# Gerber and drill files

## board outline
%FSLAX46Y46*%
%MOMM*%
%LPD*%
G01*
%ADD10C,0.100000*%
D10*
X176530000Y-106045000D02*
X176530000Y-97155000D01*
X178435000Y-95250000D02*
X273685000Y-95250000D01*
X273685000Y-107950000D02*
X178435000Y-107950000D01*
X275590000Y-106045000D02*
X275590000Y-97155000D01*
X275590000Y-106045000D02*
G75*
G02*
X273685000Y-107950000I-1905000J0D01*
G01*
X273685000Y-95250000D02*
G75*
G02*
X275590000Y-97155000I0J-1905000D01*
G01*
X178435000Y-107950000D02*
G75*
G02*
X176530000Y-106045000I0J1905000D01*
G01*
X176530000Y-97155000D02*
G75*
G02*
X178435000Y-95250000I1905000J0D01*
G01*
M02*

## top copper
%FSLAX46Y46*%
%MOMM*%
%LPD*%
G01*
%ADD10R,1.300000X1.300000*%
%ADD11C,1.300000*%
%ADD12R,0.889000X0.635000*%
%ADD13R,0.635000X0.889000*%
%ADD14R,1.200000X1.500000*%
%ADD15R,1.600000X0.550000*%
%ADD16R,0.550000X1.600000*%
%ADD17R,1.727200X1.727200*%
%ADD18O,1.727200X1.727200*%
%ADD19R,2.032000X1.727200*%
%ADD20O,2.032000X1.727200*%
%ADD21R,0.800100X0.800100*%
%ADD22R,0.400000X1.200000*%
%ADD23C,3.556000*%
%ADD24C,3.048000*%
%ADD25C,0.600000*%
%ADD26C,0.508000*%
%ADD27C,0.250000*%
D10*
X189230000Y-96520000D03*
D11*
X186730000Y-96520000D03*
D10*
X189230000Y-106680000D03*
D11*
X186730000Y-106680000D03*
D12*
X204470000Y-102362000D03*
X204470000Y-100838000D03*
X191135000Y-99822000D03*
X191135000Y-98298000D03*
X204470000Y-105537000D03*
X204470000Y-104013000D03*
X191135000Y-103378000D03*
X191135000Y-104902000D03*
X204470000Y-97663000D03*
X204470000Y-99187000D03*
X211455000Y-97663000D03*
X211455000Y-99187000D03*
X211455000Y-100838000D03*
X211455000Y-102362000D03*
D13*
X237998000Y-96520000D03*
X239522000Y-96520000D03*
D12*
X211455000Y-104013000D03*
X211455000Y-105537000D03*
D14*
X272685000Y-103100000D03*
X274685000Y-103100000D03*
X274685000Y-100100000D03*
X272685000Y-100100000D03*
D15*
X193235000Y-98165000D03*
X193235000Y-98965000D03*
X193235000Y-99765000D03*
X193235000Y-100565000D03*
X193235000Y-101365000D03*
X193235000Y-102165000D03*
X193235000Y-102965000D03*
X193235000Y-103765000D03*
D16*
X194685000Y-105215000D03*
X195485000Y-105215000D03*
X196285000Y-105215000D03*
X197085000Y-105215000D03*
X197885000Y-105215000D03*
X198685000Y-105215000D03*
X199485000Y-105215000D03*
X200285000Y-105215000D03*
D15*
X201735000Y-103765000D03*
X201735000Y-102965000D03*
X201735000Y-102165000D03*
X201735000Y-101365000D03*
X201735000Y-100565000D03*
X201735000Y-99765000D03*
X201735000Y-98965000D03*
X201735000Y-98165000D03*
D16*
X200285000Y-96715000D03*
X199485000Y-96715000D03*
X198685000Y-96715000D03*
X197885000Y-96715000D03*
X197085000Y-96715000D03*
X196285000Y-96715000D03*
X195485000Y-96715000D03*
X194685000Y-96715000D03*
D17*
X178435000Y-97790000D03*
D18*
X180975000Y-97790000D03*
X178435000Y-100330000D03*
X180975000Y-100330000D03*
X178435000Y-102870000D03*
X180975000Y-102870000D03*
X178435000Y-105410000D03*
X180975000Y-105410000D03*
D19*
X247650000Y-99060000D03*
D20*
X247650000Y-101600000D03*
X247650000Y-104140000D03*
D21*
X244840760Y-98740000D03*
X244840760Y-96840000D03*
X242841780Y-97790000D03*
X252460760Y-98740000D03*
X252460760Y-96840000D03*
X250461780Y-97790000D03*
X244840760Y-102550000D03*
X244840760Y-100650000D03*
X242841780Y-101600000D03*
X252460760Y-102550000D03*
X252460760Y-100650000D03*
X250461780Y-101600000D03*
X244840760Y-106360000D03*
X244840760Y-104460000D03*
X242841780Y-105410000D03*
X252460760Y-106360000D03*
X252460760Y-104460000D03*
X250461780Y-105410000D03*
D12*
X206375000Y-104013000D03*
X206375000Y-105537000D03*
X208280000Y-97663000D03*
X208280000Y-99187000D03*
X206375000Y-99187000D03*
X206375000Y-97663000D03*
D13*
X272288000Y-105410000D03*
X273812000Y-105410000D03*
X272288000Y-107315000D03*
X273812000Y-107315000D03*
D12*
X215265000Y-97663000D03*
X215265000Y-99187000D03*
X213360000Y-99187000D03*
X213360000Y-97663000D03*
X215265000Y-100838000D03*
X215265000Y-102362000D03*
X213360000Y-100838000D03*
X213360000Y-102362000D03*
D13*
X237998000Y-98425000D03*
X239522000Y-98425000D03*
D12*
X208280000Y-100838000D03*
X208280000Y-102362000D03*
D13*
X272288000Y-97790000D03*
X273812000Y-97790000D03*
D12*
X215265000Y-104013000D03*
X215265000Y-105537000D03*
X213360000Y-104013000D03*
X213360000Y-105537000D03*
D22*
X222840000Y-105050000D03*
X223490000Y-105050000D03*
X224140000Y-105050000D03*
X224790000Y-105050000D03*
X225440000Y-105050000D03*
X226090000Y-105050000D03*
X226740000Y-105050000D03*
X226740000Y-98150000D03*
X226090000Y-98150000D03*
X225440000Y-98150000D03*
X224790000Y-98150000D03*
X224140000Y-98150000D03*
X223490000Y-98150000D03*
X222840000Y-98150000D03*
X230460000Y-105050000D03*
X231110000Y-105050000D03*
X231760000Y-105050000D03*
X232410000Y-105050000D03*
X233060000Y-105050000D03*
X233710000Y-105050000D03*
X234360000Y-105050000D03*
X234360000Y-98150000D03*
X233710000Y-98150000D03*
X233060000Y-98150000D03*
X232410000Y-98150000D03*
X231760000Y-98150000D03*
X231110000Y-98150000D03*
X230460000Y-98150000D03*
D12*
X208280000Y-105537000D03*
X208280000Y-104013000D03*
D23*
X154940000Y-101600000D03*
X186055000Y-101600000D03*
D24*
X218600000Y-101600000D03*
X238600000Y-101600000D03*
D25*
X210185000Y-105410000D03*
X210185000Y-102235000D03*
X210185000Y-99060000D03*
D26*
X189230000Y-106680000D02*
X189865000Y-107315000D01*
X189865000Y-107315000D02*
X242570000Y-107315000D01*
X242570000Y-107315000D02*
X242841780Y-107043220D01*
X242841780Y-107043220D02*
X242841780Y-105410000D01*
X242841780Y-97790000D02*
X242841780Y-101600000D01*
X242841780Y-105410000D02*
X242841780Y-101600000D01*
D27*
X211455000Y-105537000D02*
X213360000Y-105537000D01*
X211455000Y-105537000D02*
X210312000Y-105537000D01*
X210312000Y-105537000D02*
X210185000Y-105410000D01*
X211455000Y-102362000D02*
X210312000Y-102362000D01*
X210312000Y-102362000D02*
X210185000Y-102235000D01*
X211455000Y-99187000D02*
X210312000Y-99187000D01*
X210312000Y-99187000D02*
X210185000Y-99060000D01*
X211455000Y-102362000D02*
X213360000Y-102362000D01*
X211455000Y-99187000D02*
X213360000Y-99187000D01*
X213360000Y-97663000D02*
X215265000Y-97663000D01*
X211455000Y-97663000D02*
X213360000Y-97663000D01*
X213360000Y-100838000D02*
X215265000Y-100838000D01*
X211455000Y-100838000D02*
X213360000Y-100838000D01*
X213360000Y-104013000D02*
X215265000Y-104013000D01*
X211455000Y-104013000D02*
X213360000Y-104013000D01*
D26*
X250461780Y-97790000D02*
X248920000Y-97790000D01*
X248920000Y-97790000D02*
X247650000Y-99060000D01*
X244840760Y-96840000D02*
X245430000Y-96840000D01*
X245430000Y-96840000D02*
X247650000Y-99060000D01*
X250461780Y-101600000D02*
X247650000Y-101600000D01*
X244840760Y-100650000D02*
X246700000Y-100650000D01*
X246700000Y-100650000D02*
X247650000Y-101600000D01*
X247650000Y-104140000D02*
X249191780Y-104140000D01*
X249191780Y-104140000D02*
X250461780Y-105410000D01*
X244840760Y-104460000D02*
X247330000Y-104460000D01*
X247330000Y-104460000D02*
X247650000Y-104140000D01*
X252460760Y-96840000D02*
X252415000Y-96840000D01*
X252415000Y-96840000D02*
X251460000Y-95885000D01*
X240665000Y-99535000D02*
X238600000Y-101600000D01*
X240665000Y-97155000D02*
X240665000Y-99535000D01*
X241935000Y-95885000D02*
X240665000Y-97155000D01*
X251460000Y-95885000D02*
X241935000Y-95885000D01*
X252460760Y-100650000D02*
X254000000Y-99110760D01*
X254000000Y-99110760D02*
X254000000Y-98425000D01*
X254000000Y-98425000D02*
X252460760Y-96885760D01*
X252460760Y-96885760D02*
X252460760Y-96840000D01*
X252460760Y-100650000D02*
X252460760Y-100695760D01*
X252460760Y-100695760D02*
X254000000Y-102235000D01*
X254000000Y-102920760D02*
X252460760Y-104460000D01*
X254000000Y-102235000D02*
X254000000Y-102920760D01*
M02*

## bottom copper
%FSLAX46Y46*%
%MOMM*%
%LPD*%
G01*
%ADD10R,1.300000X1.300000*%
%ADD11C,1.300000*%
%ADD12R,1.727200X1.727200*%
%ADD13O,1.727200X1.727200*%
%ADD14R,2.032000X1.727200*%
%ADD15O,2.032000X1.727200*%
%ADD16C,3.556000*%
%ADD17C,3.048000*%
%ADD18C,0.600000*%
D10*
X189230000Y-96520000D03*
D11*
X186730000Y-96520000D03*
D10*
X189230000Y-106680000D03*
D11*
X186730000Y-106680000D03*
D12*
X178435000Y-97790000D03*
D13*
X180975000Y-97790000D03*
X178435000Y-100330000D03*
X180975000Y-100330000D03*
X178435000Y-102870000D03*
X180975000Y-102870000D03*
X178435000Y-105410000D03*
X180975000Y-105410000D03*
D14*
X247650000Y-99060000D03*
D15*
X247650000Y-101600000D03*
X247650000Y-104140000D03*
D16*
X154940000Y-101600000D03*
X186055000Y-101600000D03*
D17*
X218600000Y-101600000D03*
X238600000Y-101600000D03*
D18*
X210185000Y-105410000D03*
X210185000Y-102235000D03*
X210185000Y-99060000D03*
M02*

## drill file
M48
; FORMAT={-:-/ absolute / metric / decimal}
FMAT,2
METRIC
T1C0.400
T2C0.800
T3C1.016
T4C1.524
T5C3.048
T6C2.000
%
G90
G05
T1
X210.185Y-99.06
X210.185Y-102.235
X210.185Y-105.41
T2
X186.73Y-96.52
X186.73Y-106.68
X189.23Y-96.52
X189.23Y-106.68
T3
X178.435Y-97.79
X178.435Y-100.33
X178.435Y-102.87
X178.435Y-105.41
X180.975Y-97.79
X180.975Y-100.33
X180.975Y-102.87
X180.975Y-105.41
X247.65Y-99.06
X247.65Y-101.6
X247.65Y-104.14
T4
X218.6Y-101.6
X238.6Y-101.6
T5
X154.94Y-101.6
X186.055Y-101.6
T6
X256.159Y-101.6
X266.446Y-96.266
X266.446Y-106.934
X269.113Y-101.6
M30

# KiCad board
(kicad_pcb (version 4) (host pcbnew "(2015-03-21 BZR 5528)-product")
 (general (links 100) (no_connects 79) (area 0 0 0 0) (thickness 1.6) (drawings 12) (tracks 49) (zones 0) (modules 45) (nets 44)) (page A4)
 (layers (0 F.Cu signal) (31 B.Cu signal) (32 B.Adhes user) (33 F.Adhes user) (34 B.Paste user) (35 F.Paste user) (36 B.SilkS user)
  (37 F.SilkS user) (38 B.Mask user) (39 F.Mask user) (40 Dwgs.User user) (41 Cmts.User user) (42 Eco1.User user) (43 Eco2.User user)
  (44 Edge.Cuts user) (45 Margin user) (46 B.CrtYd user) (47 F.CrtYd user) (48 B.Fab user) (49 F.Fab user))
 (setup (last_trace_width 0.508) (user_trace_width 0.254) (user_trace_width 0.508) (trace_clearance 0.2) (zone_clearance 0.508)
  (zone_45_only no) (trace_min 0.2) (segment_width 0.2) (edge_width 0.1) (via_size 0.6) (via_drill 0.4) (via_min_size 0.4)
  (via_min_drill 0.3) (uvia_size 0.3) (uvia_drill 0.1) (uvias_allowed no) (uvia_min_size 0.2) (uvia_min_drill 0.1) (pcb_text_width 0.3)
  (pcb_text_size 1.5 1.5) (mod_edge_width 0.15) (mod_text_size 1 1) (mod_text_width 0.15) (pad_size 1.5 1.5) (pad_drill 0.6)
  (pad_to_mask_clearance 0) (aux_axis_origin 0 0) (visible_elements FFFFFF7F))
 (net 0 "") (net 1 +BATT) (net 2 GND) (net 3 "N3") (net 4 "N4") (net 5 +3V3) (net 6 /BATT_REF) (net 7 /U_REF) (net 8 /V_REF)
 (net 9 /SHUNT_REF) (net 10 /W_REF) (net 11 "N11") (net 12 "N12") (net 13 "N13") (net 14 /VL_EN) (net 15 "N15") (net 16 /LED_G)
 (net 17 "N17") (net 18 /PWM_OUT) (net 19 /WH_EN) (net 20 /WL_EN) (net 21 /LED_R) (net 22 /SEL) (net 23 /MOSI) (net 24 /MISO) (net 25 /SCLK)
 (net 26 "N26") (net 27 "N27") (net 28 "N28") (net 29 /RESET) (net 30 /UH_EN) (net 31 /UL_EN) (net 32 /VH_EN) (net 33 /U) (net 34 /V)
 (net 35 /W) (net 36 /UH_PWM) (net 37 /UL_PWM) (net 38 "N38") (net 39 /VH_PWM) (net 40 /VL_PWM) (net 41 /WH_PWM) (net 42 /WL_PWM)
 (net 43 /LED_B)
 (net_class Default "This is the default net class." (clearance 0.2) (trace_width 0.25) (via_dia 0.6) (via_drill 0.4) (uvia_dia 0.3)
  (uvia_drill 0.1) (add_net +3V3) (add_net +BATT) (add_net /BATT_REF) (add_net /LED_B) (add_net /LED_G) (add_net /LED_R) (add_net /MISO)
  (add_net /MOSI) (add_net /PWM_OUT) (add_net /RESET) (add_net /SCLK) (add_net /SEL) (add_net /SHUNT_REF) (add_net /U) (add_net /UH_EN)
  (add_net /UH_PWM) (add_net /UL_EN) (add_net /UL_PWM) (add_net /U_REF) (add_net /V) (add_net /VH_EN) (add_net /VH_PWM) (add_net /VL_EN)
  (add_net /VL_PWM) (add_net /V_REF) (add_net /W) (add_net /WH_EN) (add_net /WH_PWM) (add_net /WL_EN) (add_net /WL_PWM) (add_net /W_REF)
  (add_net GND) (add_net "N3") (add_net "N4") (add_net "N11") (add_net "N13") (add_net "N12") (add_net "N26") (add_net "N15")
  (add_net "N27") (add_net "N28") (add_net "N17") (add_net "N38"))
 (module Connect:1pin (layer F.Cu) (at 266.446 96.266)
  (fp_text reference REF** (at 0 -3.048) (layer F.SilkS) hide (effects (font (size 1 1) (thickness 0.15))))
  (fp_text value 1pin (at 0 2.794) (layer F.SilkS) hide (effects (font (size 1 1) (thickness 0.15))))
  (pad "" np_thru_hole circle (at 0 0) (size 2 2) (drill 2) (layers *.Cu *.Mask F.SilkS)))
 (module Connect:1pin (layer F.Cu) (at 266.446 106.934)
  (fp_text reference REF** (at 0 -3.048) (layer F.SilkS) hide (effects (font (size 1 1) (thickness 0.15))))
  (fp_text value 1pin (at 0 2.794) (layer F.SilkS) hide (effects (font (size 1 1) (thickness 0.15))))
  (pad "" np_thru_hole circle (at 0 0) (size 2 2) (drill 2) (layers *.Cu *.Mask F.SilkS)))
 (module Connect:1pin (layer F.Cu) (at 256.159 101.6)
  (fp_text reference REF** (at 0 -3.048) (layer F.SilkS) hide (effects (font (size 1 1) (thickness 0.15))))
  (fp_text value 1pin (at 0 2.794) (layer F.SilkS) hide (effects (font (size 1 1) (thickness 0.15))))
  (pad "" np_thru_hole circle (at 0 0) (size 2 2) (drill 2) (layers *.Cu *.Mask F.SilkS)))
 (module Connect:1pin (layer F.Cu) (at 269.113 101.6)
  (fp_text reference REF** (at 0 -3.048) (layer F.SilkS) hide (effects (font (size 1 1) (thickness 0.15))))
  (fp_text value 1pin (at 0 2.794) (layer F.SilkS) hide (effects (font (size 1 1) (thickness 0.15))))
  (pad "" np_thru_hole circle (at 0 0) (size 2 2) (drill 2) (layers *.Cu *.Mask F.SilkS)))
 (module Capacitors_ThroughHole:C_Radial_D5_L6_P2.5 (layer F.Cu) (at 189.23 96.52 180)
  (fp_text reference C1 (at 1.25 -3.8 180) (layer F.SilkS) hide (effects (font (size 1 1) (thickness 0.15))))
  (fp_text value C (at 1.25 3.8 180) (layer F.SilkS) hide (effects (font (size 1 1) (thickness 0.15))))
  (pad 1 thru_hole rect (at 0 0 180) (size 1.3 1.3) (drill 0.8) (layers *.Cu *.Mask F.SilkS) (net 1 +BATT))
  (pad 2 thru_hole circle (at 2.5 0 180) (size 1.3 1.3) (drill 0.8) (layers *.Cu *.Mask F.SilkS) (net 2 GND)))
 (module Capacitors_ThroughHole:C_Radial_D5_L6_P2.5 (layer F.Cu) (at 189.23 106.68 180)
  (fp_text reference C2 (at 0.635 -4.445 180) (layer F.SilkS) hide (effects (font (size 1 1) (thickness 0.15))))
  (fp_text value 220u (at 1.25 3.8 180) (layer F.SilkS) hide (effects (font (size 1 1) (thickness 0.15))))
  (pad 1 thru_hole rect (at 0 0 180) (size 1.3 1.3) (drill 0.8) (layers *.Cu *.Mask F.SilkS) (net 1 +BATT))
  (pad 2 thru_hole circle (at 2.5 0 180) (size 1.3 1.3) (drill 0.8) (layers *.Cu *.Mask F.SilkS) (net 2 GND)))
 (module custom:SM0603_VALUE (layer F.Cu) (at 204.47 101.6 90)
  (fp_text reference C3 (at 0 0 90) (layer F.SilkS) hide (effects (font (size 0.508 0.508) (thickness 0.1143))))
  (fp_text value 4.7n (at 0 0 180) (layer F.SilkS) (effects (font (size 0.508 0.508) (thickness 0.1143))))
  (pad 1 smd rect (at -0.762 0 90) (size 0.635 0.889) (layers F.Cu F.Paste F.Mask) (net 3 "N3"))
  (pad 2 smd rect (at 0.762 0 90) (size 0.635 0.889) (layers F.Cu F.Paste F.Mask) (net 2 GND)))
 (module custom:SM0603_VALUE (layer F.Cu) (at 191.135 99.06 90)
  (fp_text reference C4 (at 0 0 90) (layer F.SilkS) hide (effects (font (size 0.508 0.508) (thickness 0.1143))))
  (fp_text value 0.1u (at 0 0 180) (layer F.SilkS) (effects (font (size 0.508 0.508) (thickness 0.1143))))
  (pad 1 smd rect (at -0.762 0 90) (size 0.635 0.889) (layers F.Cu F.Paste F.Mask) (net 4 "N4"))
  (pad 2 smd rect (at 0.762 0 90) (size 0.635 0.889) (layers F.Cu F.Paste F.Mask) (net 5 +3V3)))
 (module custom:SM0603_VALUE (layer F.Cu) (at 204.47 104.775 90)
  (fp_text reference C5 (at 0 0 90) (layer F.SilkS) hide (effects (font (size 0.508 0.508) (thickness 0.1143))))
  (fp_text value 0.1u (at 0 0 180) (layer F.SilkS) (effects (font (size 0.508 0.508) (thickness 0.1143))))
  (pad 1 smd rect (at -0.762 0 90) (size 0.635 0.889) (layers F.Cu F.Paste F.Mask) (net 4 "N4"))
  (pad 2 smd rect (at 0.762 0 90) (size 0.635 0.889) (layers F.Cu F.Paste F.Mask) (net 5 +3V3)))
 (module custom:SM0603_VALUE (layer F.Cu) (at 191.135 104.14 270)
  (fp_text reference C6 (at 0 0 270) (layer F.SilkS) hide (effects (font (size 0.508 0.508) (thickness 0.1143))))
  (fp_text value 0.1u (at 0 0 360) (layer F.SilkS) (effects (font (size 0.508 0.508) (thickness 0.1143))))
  (pad 1 smd rect (at -0.762 0 270) (size 0.635 0.889) (layers F.Cu F.Paste F.Mask) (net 4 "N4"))
  (pad 2 smd rect (at 0.762 0 270) (size 0.635 0.889) (layers F.Cu F.Paste F.Mask) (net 5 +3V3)))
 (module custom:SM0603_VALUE (layer F.Cu) (at 204.47 98.425 270)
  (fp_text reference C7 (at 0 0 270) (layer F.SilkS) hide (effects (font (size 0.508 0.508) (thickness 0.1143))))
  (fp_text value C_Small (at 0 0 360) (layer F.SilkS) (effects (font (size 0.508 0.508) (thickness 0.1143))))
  (pad 1 smd rect (at -0.762 0 270) (size 0.635 0.889) (layers F.Cu F.Paste F.Mask) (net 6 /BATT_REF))
  (pad 2 smd rect (at 0.762 0 270) (size 0.635 0.889) (layers F.Cu F.Paste F.Mask) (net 2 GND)))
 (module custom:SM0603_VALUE (layer F.Cu) (at 211.455 98.425 270)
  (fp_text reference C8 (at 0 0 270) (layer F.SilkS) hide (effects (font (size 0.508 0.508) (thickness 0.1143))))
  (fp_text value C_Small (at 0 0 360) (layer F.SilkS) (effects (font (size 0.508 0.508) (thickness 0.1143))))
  (pad 1 smd rect (at -0.762 0 270) (size 0.635 0.889) (layers F.Cu F.Paste F.Mask) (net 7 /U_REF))
  (pad 2 smd rect (at 0.762 0 270) (size 0.635 0.889) (layers F.Cu F.Paste F.Mask) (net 2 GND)))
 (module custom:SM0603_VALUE (layer F.Cu) (at 211.455 101.6 270)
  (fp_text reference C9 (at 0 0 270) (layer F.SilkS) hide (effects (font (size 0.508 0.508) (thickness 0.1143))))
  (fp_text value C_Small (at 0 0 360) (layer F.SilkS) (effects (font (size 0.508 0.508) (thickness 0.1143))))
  (pad 1 smd rect (at -0.762 0 270) (size 0.635 0.889) (layers F.Cu F.Paste F.Mask) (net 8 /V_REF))
  (pad 2 smd rect (at 0.762 0 270) (size 0.635 0.889) (layers F.Cu F.Paste F.Mask) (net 2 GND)))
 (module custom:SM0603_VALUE (layer F.Cu) (at 238.76 96.52)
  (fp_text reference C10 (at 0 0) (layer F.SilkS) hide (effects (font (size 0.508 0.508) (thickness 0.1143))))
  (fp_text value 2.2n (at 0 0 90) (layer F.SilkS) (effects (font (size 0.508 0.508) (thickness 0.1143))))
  (pad 1 smd rect (at -0.762 0) (size 0.635 0.889) (layers F.Cu F.Paste F.Mask) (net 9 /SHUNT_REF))
  (pad 2 smd rect (at 0.762 0) (size 0.635 0.889) (layers F.Cu F.Paste F.Mask) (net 2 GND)))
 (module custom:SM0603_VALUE (layer F.Cu) (at 211.455 104.775 270)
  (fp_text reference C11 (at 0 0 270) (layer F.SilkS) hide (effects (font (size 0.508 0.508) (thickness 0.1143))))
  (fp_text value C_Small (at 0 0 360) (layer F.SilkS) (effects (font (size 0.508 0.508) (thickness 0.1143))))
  (pad 1 smd rect (at -0.762 0 270) (size 0.635 0.889) (layers F.Cu F.Paste F.Mask) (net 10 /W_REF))
  (pad 2 smd rect (at 0.762 0 270) (size 0.635 0.889) (layers F.Cu F.Paste F.Mask) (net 2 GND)))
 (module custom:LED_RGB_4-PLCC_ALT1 (layer F.Cu) (at 273.685 101.6 90)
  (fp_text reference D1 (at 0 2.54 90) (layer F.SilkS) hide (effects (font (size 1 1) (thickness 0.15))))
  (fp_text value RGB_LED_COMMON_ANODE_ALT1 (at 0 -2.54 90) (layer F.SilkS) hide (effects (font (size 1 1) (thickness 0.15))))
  (pad 2 smd rect (at -1.5 -1 90) (size 1.5 1.2) (layers F.Cu F.Paste F.Mask) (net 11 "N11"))
  (pad 4 smd rect (at -1.5 1 90) (size 1.5 1.2) (layers F.Cu F.Paste F.Mask) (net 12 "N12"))
  (pad 3 smd rect (at 1.5 1 90) (size 1.5 1.2) (layers F.Cu F.Paste F.Mask) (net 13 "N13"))
  (pad 1 smd rect (at 1.5 -1 90) (size 1.5 1.2) (layers F.Cu F.Paste F.Mask) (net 5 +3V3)))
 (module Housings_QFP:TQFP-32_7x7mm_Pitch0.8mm (layer F.Cu) (at 197.485 100.965)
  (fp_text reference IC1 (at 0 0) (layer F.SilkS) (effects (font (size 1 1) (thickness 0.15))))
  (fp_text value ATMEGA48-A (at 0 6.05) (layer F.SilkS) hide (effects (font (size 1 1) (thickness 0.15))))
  (pad 1 smd rect (at -4.25 -2.8) (size 1.6 0.55) (layers F.Cu F.Paste F.Mask) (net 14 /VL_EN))
  (pad 2 smd rect (at -4.25 -2) (size 1.6 0.55) (layers F.Cu F.Paste F.Mask) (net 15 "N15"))
  (pad 3 smd rect (at -4.25 -1.2) (size 1.6 0.55) (layers F.Cu F.Paste F.Mask) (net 2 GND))
  (pad 4 smd rect (at -4.25 -0.4) (size 1.6 0.55) (layers F.Cu F.Paste F.Mask) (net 4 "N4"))
  (pad 5 smd rect (at -4.25 0.4) (size 1.6 0.55) (layers F.Cu F.Paste F.Mask) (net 2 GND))
  (pad 6 smd rect (at -4.25 1.2) (size 1.6 0.55) (layers F.Cu F.Paste F.Mask) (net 4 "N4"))
  (pad 7 smd rect (at -4.25 2) (size 1.6 0.55) (layers F.Cu F.Paste F.Mask) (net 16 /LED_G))
  (pad 8 smd rect (at -4.25 2.8) (size 1.6 0.55) (layers F.Cu F.Paste F.Mask) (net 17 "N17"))
  (pad 9 smd rect (at -2.8 4.25 90) (size 1.6 0.55) (layers F.Cu F.Paste F.Mask) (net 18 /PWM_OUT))
  (pad 10 smd rect (at -2 4.25 90) (size 1.6 0.55) (layers F.Cu F.Paste F.Mask) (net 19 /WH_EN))
  (pad 11 smd rect (at -1.2 4.25 90) (size 1.6 0.55) (layers F.Cu F.Paste F.Mask) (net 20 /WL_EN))
  (pad 12 smd rect (at -0.4 4.25 90) (size 1.6 0.55) (layers F.Cu F.Paste F.Mask) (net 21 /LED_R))
  (pad 13 smd rect (at 0.4 4.25 90) (size 1.6 0.55) (layers F.Cu F.Paste F.Mask) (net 16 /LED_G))
  (pad 14 smd rect (at 1.2 4.25 90) (size 1.6 0.55) (layers F.Cu F.Paste F.Mask) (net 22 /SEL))
  (pad 15 smd rect (at 2 4.25 90) (size 1.6 0.55) (layers F.Cu F.Paste F.Mask) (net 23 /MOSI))
  (pad 16 smd rect (at 2.8 4.25 90) (size 1.6 0.55) (layers F.Cu F.Paste F.Mask) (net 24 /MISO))
  (pad 17 smd rect (at 4.25 2.8) (size 1.6 0.55) (layers F.Cu F.Paste F.Mask) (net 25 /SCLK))
  (pad 18 smd rect (at 4.25 2) (size 1.6 0.55) (layers F.Cu F.Paste F.Mask) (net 4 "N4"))
  (pad 19 smd rect (at 4.25 1.2) (size 1.6 0.55) (layers F.Cu F.Paste F.Mask) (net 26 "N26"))
  (pad 20 smd rect (at 4.25 0.4) (size 1.6 0.55) (layers F.Cu F.Paste F.Mask) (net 3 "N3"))
  (pad 21 smd rect (at 4.25 -0.4) (size 1.6 0.55) (layers F.Cu F.Paste F.Mask) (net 2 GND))
  (pad 22 smd rect (at 4.25 -1.2) (size 1.6 0.55) (layers F.Cu F.Paste F.Mask) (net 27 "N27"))
  (pad 23 smd rect (at 4.25 -2) (size 1.6 0.55) (layers F.Cu F.Paste F.Mask) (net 7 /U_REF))
  (pad 24 smd rect (at 4.25 -2.8) (size 1.6 0.55) (layers F.Cu F.Paste F.Mask) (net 8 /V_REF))
  (pad 25 smd rect (at 2.8 -4.25 90) (size 1.6 0.55) (layers F.Cu F.Paste F.Mask) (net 10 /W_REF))
  (pad 26 smd rect (at 2 -4.25 90) (size 1.6 0.55) (layers F.Cu F.Paste F.Mask) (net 9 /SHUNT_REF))
  (pad 27 smd rect (at 1.2 -4.25 90) (size 1.6 0.55) (layers F.Cu F.Paste F.Mask) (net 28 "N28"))
  (pad 28 smd rect (at 0.4 -4.25 90) (size 1.6 0.55) (layers F.Cu F.Paste F.Mask) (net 6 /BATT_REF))
  (pad 29 smd rect (at -0.4 -4.25 90) (size 1.6 0.55) (layers F.Cu F.Paste F.Mask) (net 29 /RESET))
  (pad 30 smd rect (at -1.2 -4.25 90) (size 1.6 0.55) (layers F.Cu F.Paste F.Mask) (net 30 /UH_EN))
  (pad 31 smd rect (at -2 -4.25 90) (size 1.6 0.55) (layers F.Cu F.Paste F.Mask) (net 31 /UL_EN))
  (pad 32 smd rect (at -2.8 -4.25 90) (size 1.6 0.55) (layers F.Cu F.Paste F.Mask) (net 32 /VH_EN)))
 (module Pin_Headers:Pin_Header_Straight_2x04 (layer F.Cu) (at 178.435 97.79)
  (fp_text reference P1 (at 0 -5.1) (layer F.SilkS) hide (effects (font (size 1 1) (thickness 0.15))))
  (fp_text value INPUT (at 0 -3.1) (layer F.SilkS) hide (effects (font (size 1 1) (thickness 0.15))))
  (pad 1 thru_hole rect (at 0 0) (size 1.7272 1.7272) (drill 1.016) (layers *.Cu *.Mask F.SilkS) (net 24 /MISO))
  (pad 2 thru_hole oval (at 2.54 0) (size 1.7272 1.7272) (drill 1.016) (layers *.Cu *.Mask F.SilkS) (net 5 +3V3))
  (pad 3 thru_hole oval (at 0 2.54) (size 1.7272 1.7272) (drill 1.016) (layers *.Cu *.Mask F.SilkS) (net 25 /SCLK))
  (pad 4 thru_hole oval (at 2.54 2.54) (size 1.7272 1.7272) (drill 1.016) (layers *.Cu *.Mask F.SilkS) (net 23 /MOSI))
  (pad 5 thru_hole oval (at 0 5.08) (size 1.7272 1.7272) (drill 1.016) (layers *.Cu *.Mask F.SilkS) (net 29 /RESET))
  (pad 6 thru_hole oval (at 2.54 5.08) (size 1.7272 1.7272) (drill 1.016) (layers *.Cu *.Mask F.SilkS) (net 2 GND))
  (pad 7 thru_hole oval (at 0 7.62) (size 1.7272 1.7272) (drill 1.016) (layers *.Cu *.Mask F.SilkS) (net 22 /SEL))
  (pad 8 thru_hole oval (at 2.54 7.62) (size 1.7272 1.7272) (drill 1.016) (layers *.Cu *.Mask F.SilkS) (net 1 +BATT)))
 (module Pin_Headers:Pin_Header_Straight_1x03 (layer F.Cu) (at 247.65 99.06)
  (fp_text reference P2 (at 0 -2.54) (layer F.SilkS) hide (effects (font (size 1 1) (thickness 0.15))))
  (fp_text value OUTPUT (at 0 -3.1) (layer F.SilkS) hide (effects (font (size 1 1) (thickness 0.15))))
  (pad 1 thru_hole rect (at 0 0) (size 2.032 1.7272) (drill 1.016) (layers *.Cu *.Mask F.SilkS) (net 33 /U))
  (pad 2 thru_hole oval (at 0 2.54) (size 2.032 1.7272) (drill 1.016) (layers *.Cu *.Mask F.SilkS) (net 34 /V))
  (pad 3 thru_hole oval (at 0 5.08) (size 2.032 1.7272) (drill 1.016) (layers *.Cu *.Mask F.SilkS) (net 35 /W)))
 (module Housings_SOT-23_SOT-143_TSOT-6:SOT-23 (layer F.Cu) (at 243.84 97.79 90)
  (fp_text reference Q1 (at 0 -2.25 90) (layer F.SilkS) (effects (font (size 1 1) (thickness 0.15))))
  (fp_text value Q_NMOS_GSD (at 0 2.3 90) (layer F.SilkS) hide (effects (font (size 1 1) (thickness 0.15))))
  (pad 1 smd rect (at -0.95 1.00076 90) (size 0.8001 0.8001) (layers F.Cu F.Paste F.Mask) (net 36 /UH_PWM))
  (pad 2 smd rect (at 0.95 1.00076 90) (size 0.8001 0.8001) (layers F.Cu F.Paste F.Mask) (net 33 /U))
  (pad 3 smd rect (at 0 -0.99822 90) (size 0.8001 0.8001) (layers F.Cu F.Paste F.Mask) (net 1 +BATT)))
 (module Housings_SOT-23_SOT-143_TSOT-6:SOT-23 (layer F.Cu) (at 251.46 97.79 90)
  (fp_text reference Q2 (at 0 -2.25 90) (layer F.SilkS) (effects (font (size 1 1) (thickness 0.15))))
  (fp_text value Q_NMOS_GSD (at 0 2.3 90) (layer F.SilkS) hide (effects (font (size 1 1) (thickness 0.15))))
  (pad 1 smd rect (at -0.95 1.00076 90) (size 0.8001 0.8001) (layers F.Cu F.Paste F.Mask) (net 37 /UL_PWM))
  (pad 2 smd rect (at 0.95 1.00076 90) (size 0.8001 0.8001) (layers F.Cu F.Paste F.Mask) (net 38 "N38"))
  (pad 3 smd rect (at 0 -0.99822 90) (size 0.8001 0.8001) (layers F.Cu F.Paste F.Mask) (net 33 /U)))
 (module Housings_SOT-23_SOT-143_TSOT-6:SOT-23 (layer F.Cu) (at 243.84 101.6 90)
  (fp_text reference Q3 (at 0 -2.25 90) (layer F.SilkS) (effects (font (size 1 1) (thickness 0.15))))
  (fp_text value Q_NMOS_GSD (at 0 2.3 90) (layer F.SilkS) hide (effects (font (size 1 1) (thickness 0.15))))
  (pad 1 smd rect (at -0.95 1.00076 90) (size 0.8001 0.8001) (layers F.Cu F.Paste F.Mask) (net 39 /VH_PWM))
  (pad 2 smd rect (at 0.95 1.00076 90) (size 0.8001 0.8001) (layers F.Cu F.Paste F.Mask) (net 34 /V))
  (pad 3 smd rect (at 0 -0.99822 90) (size 0.8001 0.8001) (layers F.Cu F.Paste F.Mask) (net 1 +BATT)))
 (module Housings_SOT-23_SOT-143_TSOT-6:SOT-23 (layer F.Cu) (at 251.46 101.6 90)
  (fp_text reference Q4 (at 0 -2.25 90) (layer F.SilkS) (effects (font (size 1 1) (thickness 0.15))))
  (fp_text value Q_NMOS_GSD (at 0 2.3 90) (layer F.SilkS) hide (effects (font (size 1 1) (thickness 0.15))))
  (pad 1 smd rect (at -0.95 1.00076 90) (size 0.8001 0.8001) (layers F.Cu F.Paste F.Mask) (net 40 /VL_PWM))
  (pad 2 smd rect (at 0.95 1.00076 90) (size 0.8001 0.8001) (layers F.Cu F.Paste F.Mask) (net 38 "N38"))
  (pad 3 smd rect (at 0 -0.99822 90) (size 0.8001 0.8001) (layers F.Cu F.Paste F.Mask) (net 34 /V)))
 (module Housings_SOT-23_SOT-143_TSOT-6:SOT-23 (layer F.Cu) (at 243.84 105.41 90)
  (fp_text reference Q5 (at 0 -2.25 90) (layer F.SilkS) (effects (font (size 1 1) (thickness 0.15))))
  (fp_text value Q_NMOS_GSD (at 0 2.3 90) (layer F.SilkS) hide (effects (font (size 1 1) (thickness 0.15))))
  (pad 1 smd rect (at -0.95 1.00076 90) (size 0.8001 0.8001) (layers F.Cu F.Paste F.Mask) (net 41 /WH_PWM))
  (pad 2 smd rect (at 0.95 1.00076 90) (size 0.8001 0.8001) (layers F.Cu F.Paste F.Mask) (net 35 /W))
  (pad 3 smd rect (at 0 -0.99822 90) (size 0.8001 0.8001) (layers F.Cu F.Paste F.Mask) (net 1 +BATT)))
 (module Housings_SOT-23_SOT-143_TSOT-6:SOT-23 (layer F.Cu) (at 251.46 105.41 90)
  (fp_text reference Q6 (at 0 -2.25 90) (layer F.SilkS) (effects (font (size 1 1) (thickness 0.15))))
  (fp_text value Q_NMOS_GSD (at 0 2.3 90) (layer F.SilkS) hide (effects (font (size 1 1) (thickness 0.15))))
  (pad 1 smd rect (at -0.95 1.00076 90) (size 0.8001 0.8001) (layers F.Cu F.Paste F.Mask) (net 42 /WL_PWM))
  (pad 2 smd rect (at 0.95 1.00076 90) (size 0.8001 0.8001) (layers F.Cu F.Paste F.Mask) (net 38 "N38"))
  (pad 3 smd rect (at 0 -0.99822 90) (size 0.8001 0.8001) (layers F.Cu F.Paste F.Mask) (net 35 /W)))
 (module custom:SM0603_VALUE (layer F.Cu) (at 206.375 104.775 270)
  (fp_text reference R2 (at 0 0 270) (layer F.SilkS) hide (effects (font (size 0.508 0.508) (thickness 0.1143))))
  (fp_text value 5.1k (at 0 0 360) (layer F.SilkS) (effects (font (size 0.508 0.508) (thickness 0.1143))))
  (pad 1 smd rect (at -0.762 0 270) (size 0.635 0.889) (layers F.Cu F.Paste F.Mask) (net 3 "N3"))
  (pad 2 smd rect (at 0.762 0 270) (size 0.635 0.889) (layers F.Cu F.Paste F.Mask) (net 2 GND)))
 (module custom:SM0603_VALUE (layer F.Cu) (at 208.28 98.425 270)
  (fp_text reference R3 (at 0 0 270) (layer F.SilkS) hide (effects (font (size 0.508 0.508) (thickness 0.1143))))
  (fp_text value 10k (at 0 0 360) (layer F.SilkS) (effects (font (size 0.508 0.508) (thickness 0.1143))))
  (pad 1 smd rect (at -0.762 0 270) (size 0.635 0.889) (layers F.Cu F.Paste F.Mask) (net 6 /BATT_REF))
  (pad 2 smd rect (at 0.762 0 270) (size 0.635 0.889) (layers F.Cu F.Paste F.Mask) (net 1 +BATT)))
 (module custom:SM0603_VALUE (layer F.Cu) (at 206.375 98.425 90)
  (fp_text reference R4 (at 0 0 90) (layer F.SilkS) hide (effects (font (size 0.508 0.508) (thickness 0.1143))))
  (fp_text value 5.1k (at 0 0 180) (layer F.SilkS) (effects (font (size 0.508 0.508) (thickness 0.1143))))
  (pad 1 smd rect (at -0.762 0 90) (size 0.635 0.889) (layers F.Cu F.Paste F.Mask) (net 2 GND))
  (pad 2 smd rect (at 0.762 0 90) (size 0.635 0.889) (layers F.Cu F.Paste F.Mask) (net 6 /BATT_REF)))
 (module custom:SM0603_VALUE (layer F.Cu) (at 273.05 105.41)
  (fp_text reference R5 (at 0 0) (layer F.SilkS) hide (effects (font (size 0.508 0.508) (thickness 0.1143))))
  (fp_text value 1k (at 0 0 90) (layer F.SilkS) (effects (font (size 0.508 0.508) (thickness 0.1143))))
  (pad 1 smd rect (at -0.762 0) (size 0.635 0.889) (layers F.Cu F.Paste F.Mask) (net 21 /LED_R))
  (pad 2 smd rect (at 0.762 0) (size 0.635 0.889) (layers F.Cu F.Paste F.Mask) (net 11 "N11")))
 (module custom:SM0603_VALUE (layer F.Cu) (at 273.05 107.315)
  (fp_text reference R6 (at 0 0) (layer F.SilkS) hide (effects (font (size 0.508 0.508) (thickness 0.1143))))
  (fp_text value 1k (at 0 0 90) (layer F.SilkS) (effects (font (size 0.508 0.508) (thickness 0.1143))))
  (pad 1 smd rect (at -0.762 0) (size 0.635 0.889) (layers F.Cu F.Paste F.Mask) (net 16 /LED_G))
  (pad 2 smd rect (at 0.762 0) (size 0.635 0.889) (layers F.Cu F.Paste F.Mask) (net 12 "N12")))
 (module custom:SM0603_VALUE (layer F.Cu) (at 215.265 98.425 270)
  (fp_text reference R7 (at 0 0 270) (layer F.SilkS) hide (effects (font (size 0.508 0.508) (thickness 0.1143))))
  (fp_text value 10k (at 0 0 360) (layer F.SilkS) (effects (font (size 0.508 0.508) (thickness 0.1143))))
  (pad 1 smd rect (at -0.762 0 270) (size 0.635 0.889) (layers F.Cu F.Paste F.Mask) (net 7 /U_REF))
  (pad 2 smd rect (at 0.762 0 270) (size 0.635 0.889) (layers F.Cu F.Paste F.Mask) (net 33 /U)))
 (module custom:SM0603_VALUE (layer F.Cu) (at 213.36 98.425 90)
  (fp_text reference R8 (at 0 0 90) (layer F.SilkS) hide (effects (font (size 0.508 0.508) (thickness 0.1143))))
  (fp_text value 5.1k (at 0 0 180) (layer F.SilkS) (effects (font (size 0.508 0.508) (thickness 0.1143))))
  (pad 1 smd rect (at -0.762 0 90) (size 0.635 0.889) (layers F.Cu F.Paste F.Mask) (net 2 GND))
  (pad 2 smd rect (at 0.762 0 90) (size 0.635 0.889) (layers F.Cu F.Paste F.Mask) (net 7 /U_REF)))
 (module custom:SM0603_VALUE (layer F.Cu) (at 215.265 101.6 270)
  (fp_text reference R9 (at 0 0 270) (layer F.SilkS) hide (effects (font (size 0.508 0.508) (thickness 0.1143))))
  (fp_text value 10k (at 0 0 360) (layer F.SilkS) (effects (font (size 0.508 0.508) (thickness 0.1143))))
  (pad 1 smd rect (at -0.762 0 270) (size 0.635 0.889) (layers F.Cu F.Paste F.Mask) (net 8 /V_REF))
  (pad 2 smd rect (at 0.762 0 270) (size 0.635 0.889) (layers F.Cu F.Paste F.Mask) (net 34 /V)))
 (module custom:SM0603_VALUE (layer F.Cu) (at 213.36 101.6 270)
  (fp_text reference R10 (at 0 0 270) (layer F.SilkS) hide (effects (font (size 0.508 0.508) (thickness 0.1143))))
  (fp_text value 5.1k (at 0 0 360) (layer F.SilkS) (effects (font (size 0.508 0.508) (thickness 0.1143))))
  (pad 1 smd rect (at -0.762 0 270) (size 0.635 0.889) (layers F.Cu F.Paste F.Mask) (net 8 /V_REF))
  (pad 2 smd rect (at 0.762 0 270) (size 0.635 0.889) (layers F.Cu F.Paste F.Mask) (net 2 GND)))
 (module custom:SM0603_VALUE (layer F.Cu) (at 238.76 98.425)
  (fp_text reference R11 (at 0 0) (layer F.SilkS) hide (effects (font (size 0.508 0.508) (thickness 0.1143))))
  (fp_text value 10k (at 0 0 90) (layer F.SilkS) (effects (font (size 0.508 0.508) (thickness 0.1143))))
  (pad 1 smd rect (at -0.762 0) (size 0.635 0.889) (layers F.Cu F.Paste F.Mask) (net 9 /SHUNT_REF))
  (pad 2 smd rect (at 0.762 0) (size 0.635 0.889) (layers F.Cu F.Paste F.Mask) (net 38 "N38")))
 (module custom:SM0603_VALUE (layer F.Cu) (at 208.28 101.6 270)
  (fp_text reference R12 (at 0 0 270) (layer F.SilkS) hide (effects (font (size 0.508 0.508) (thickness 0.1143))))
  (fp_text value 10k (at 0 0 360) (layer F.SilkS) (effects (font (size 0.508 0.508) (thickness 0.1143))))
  (pad 1 smd rect (at -0.762 0 270) (size 0.635 0.889) (layers F.Cu F.Paste F.Mask) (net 29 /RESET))
  (pad 2 smd rect (at 0.762 0 270) (size 0.635 0.889) (layers F.Cu F.Paste F.Mask) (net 5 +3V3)))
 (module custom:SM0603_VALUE (layer F.Cu) (at 273.05 97.79)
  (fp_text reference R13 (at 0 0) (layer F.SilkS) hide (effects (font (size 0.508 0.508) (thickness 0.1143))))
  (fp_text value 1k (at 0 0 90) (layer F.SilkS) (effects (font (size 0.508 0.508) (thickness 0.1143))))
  (pad 1 smd rect (at -0.762 0) (size 0.635 0.889) (layers F.Cu F.Paste F.Mask) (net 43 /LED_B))
  (pad 2 smd rect (at 0.762 0) (size 0.635 0.889) (layers F.Cu F.Paste F.Mask) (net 13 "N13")))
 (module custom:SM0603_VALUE (layer F.Cu) (at 215.265 104.775 270)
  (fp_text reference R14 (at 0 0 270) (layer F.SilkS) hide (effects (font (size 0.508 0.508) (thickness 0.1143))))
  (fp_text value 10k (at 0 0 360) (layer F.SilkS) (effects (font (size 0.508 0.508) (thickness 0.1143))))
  (pad 1 smd rect (at -0.762 0 270) (size 0.635 0.889) (layers F.Cu F.Paste F.Mask) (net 10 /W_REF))
  (pad 2 smd rect (at 0.762 0 270) (size 0.635 0.889) (layers F.Cu F.Paste F.Mask) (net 35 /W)))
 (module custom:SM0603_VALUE (layer F.Cu) (at 213.36 104.775 270)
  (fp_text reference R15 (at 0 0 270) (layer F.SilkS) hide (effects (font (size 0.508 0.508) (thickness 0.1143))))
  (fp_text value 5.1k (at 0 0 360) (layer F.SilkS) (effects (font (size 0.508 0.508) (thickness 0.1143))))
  (pad 1 smd rect (at -0.762 0 270) (size 0.635 0.889) (layers F.Cu F.Paste F.Mask) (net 10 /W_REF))
  (pad 2 smd rect (at 0.762 0 270) (size 0.635 0.889) (layers F.Cu F.Paste F.Mask) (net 2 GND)))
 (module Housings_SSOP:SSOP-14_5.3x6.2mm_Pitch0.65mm (layer F.Cu) (at 224.79 101.6 90)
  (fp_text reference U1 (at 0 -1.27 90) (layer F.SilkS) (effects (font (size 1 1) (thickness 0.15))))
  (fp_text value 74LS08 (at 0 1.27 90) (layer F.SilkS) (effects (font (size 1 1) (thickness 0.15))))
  (pad 1 smd rect (at -3.45 -1.95 90) (size 1.2 0.4) (layers F.Cu F.Paste F.Mask) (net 18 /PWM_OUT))
  (pad 2 smd rect (at -3.45 -1.3 90) (size 1.2 0.4) (layers F.Cu F.Paste F.Mask) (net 19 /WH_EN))
  (pad 3 smd rect (at -3.45 -0.65 90) (size 1.2 0.4) (layers F.Cu F.Paste F.Mask) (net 41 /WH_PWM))
  (pad 4 smd rect (at -3.45 0 90) (size 1.2 0.4) (layers F.Cu F.Paste F.Mask) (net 18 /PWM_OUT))
  (pad 5 smd rect (at -3.45 0.65 90) (size 1.2 0.4) (layers F.Cu F.Paste F.Mask) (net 32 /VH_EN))
  (pad 6 smd rect (at -3.45 1.3 90) (size 1.2 0.4) (layers F.Cu F.Paste F.Mask) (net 39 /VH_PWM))
  (pad 7 smd rect (at -3.45 1.95 90) (size 1.2 0.4) (layers F.Cu F.Paste F.Mask) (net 2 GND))
  (pad 8 smd rect (at 3.45 1.95 90) (size 1.2 0.4) (layers F.Cu F.Paste F.Mask) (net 36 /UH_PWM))
  (pad 9 smd rect (at 3.45 1.3 90) (size 1.2 0.4) (layers F.Cu F.Paste F.Mask) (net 18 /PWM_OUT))
  (pad 10 smd rect (at 3.45 0.65 90) (size 1.2 0.4) (layers F.Cu F.Paste F.Mask) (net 30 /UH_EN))
  (pad 11 smd rect (at 3.45 0 90) (size 1.2 0.4) (layers F.Cu F.Paste F.Mask))
  (pad 12 smd rect (at 3.45 -0.65 90) (size 1.2 0.4) (layers F.Cu F.Paste F.Mask))
  (pad 13 smd rect (at 3.45 -1.3 90) (size 1.2 0.4) (layers F.Cu F.Paste F.Mask))
  (pad 14 smd rect (at 3.45 -1.95 90) (size 1.2 0.4) (layers F.Cu F.Paste F.Mask) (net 5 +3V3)))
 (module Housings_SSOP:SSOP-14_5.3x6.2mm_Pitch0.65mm (layer F.Cu) (at 232.41 101.6 90)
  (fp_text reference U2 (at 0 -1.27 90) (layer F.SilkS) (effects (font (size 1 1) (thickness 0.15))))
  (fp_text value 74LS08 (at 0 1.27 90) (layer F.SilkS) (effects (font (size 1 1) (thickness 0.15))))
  (pad 1 smd rect (at -3.45 -1.95 90) (size 1.2 0.4) (layers F.Cu F.Paste F.Mask) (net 18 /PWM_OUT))
  (pad 2 smd rect (at -3.45 -1.3 90) (size 1.2 0.4) (layers F.Cu F.Paste F.Mask) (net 20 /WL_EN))
  (pad 3 smd rect (at -3.45 -0.65 90) (size 1.2 0.4) (layers F.Cu F.Paste F.Mask) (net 42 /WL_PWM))
  (pad 4 smd rect (at -3.45 0 90) (size 1.2 0.4) (layers F.Cu F.Paste F.Mask) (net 18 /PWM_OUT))
  (pad 5 smd rect (at -3.45 0.65 90) (size 1.2 0.4) (layers F.Cu F.Paste F.Mask) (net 14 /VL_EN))
  (pad 6 smd rect (at -3.45 1.3 90) (size 1.2 0.4) (layers F.Cu F.Paste F.Mask) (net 40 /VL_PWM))
  (pad 7 smd rect (at -3.45 1.95 90) (size 1.2 0.4) (layers F.Cu F.Paste F.Mask) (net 2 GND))
  (pad 8 smd rect (at 3.45 1.95 90) (size 1.2 0.4) (layers F.Cu F.Paste F.Mask) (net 37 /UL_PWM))
  (pad 9 smd rect (at 3.45 1.3 90) (size 1.2 0.4) (layers F.Cu F.Paste F.Mask) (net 18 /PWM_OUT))
  (pad 10 smd rect (at 3.45 0.65 90) (size 1.2 0.4) (layers F.Cu F.Paste F.Mask) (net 31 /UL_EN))
  (pad 11 smd rect (at 3.45 0 90) (size 1.2 0.4) (layers F.Cu F.Paste F.Mask))
  (pad 12 smd rect (at 3.45 -0.65 90) (size 1.2 0.4) (layers F.Cu F.Paste F.Mask))
  (pad 13 smd rect (at 3.45 -1.3 90) (size 1.2 0.4) (layers F.Cu F.Paste F.Mask))
  (pad 14 smd rect (at 3.45 -1.95 90) (size 1.2 0.4) (layers F.Cu F.Paste F.Mask) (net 5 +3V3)))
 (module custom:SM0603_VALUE (layer F.Cu) (at 208.28 104.775 90)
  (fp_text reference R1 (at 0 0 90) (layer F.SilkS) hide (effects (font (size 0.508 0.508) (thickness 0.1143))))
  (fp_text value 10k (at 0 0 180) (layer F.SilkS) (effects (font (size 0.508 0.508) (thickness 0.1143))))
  (pad 1 smd rect (at -0.762 0 90) (size 0.635 0.889) (layers F.Cu F.Paste F.Mask) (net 5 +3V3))
  (pad 2 smd rect (at 0.762 0 90) (size 0.635 0.889) (layers F.Cu F.Paste F.Mask) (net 3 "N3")))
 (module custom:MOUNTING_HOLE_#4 (layer F.Cu) (at 154.94 101.6)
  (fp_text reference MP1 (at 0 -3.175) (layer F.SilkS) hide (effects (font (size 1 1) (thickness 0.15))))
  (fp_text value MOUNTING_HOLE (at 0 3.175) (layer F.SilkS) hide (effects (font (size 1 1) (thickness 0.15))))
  (pad 1 thru_hole circle (at 0 0) (size 3.556 3.556) (drill 3.048) (layers *.Cu *.Mask F.SilkS) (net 2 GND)))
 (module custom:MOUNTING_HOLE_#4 (layer F.Cu) (at 186.055 101.6)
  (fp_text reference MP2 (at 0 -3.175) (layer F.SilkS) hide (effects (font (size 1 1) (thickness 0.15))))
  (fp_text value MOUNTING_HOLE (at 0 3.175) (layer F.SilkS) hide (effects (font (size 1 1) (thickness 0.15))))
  (pad 1 thru_hole circle (at 0 0) (size 3.556 3.556) (drill 3.048) (layers *.Cu *.Mask F.SilkS) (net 2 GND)))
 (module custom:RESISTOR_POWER (layer F.Cu) (at 228.6 101.6)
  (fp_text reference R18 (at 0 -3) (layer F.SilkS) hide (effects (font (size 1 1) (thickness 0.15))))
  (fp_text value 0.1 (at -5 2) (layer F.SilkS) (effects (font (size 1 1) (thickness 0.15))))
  (pad 1 thru_hole circle (at -10 0) (size 3.048 3.048) (drill 1.524) (layers *.Cu *.Mask F.SilkS) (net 2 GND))
  (pad 2 thru_hole circle (at 10 0) (size 3.048 3.048) (drill 1.524) (layers *.Cu *.Mask F.SilkS) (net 38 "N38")))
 (gr_line (start 176.53 106.045) (end 176.53 97.155) (angle 90) (layer Edge.Cuts) (width 0.1))
 (gr_line (start 178.435 95.25) (end 273.685 95.25) (angle 90) (layer Edge.Cuts) (width 0.1))
 (gr_line (start 273.685 107.95) (end 178.435 107.95) (angle 90) (layer Edge.Cuts) (width 0.1))
 (gr_line (start 275.59 106.045) (end 275.59 97.155) (angle 90) (layer Edge.Cuts) (width 0.1))
 (gr_arc (start 273.685 106.045) (end 275.59 106.045) (angle 90) (layer Edge.Cuts) (width 0.1))
 (gr_arc (start 273.685 97.155) (end 273.685 95.25) (angle 90) (layer Edge.Cuts) (width 0.1))
 (gr_arc (start 178.435 106.045) (end 178.435 107.95) (angle 90) (layer Edge.Cuts) (width 0.1))
 (gr_arc (start 178.435 97.155) (end 176.53 97.155) (angle 90) (layer Edge.Cuts) (width 0.1))
 (segment (start 189.23 106.68) (end 189.865 107.315) (width 0.508) (layer F.Cu) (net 1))
 (segment (start 189.865 107.315) (end 242.57 107.315) (width 0.508) (layer F.Cu) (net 1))
 (segment (start 242.57 107.315) (end 242.84178 107.04322) (width 0.508) (layer F.Cu) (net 1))
 (segment (start 242.84178 107.04322) (end 242.84178 105.41) (width 0.508) (layer F.Cu) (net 1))
 (segment (start 242.84178 97.79) (end 242.84178 101.6) (width 0.508) (layer F.Cu) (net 1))
 (segment (start 242.84178 105.41) (end 242.84178 101.6) (width 0.508) (layer F.Cu) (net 1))
 (segment (start 211.455 105.537) (end 213.36 105.537) (width 0.25) (layer F.Cu) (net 2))
 (segment (start 211.455 105.537) (end 210.312 105.537) (width 0.25) (layer F.Cu) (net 2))
 (via (at 210.185 105.41) (size 0.6) (layers F.Cu B.Cu) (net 2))
 (segment (start 210.312 105.537) (end 210.185 105.41) (width 0.25) (layer F.Cu) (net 2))
 (segment (start 211.455 102.362) (end 210.312 102.362) (width 0.25) (layer F.Cu) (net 2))
 (via (at 210.185 102.235) (size 0.6) (layers F.Cu B.Cu) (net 2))
 (segment (start 210.312 102.362) (end 210.185 102.235) (width 0.25) (layer F.Cu) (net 2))
 (segment (start 211.455 99.187) (end 210.312 99.187) (width 0.25) (layer F.Cu) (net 2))
 (via (at 210.185 99.06) (size 0.6) (layers F.Cu B.Cu) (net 2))
 (segment (start 210.312 99.187) (end 210.185 99.06) (width 0.25) (layer F.Cu) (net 2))
 (segment (start 211.455 102.362) (end 213.36 102.362) (width 0.25) (layer F.Cu) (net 2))
 (segment (start 211.455 99.187) (end 213.36 99.187) (width 0.25) (layer F.Cu) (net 2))
 (segment (start 213.36 97.663) (end 215.265 97.663) (width 0.25) (layer F.Cu) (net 7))
 (segment (start 211.455 97.663) (end 213.36 97.663) (width 0.25) (layer F.Cu) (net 7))
 (segment (start 213.36 100.838) (end 215.265 100.838) (width 0.25) (layer F.Cu) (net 8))
 (segment (start 211.455 100.838) (end 213.36 100.838) (width 0.25) (layer F.Cu) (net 8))
 (segment (start 213.36 104.013) (end 215.265 104.013) (width 0.25) (layer F.Cu) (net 10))
 (segment (start 211.455 104.013) (end 213.36 104.013) (width 0.25) (layer F.Cu) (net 10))
 (segment (start 250.46178 97.79) (end 248.92 97.79) (width 0.508) (layer F.Cu) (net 33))
 (segment (start 248.92 97.79) (end 247.65 99.06) (width 0.508) (layer F.Cu) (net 33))
 (segment (start 244.84076 96.84) (end 245.43 96.84) (width 0.508) (layer F.Cu) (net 33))
 (segment (start 245.43 96.84) (end 247.65 99.06) (width 0.508) (layer F.Cu) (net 33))
 (segment (start 250.46178 101.6) (end 247.65 101.6) (width 0.508) (layer F.Cu) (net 34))
 (segment (start 244.84076 100.65) (end 246.7 100.65) (width 0.508) (layer F.Cu) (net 34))
 (segment (start 246.7 100.65) (end 247.65 101.6) (width 0.508) (layer F.Cu) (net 34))
 (segment (start 247.65 104.14) (end 249.19178 104.14) (width 0.508) (layer F.Cu) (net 35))
 (segment (start 249.19178 104.14) (end 250.46178 105.41) (width 0.508) (layer F.Cu) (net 35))
 (segment (start 244.84076 104.46) (end 247.33 104.46) (width 0.508) (layer F.Cu) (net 35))
 (segment (start 247.33 104.46) (end 247.65 104.14) (width 0.508) (layer F.Cu) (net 35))
 (segment (start 252.46076 96.84) (end 252.415 96.84) (width 0.508) (layer F.Cu) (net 38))
 (segment (start 252.415 96.84) (end 251.46 95.885) (width 0.508) (layer F.Cu) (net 38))
 (segment (start 240.665 99.535) (end 238.6 101.6) (width 0.508) (layer F.Cu) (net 38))
 (segment (start 240.665 97.155) (end 240.665 99.535) (width 0.508) (layer F.Cu) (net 38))
 (segment (start 241.935 95.885) (end 240.665 97.155) (width 0.508) (layer F.Cu) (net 38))
 (segment (start 251.46 95.885) (end 241.935 95.885) (width 0.508) (layer F.Cu) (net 38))
 (segment (start 252.46076 100.65) (end 254 99.11076) (width 0.508) (layer F.Cu) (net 38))
 (segment (start 254 99.11076) (end 254 98.425) (width 0.508) (layer F.Cu) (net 38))
 (segment (start 254 98.425) (end 252.46076 96.88576) (width 0.508) (layer F.Cu) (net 38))
 (segment (start 252.46076 96.88576) (end 252.46076 96.84) (width 0.508) (layer F.Cu) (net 38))
 (segment (start 252.46076 100.65) (end 252.46076 100.69576) (width 0.508) (layer F.Cu) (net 38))
 (segment (start 252.46076 100.69576) (end 254 102.235) (width 0.508) (layer F.Cu) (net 38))
 (segment (start 254 102.92076) (end 252.46076 104.46) (width 0.508) (layer F.Cu) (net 38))
 (segment (start 254 102.235) (end 254 102.92076) (width 0.508) (layer F.Cu) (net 38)))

